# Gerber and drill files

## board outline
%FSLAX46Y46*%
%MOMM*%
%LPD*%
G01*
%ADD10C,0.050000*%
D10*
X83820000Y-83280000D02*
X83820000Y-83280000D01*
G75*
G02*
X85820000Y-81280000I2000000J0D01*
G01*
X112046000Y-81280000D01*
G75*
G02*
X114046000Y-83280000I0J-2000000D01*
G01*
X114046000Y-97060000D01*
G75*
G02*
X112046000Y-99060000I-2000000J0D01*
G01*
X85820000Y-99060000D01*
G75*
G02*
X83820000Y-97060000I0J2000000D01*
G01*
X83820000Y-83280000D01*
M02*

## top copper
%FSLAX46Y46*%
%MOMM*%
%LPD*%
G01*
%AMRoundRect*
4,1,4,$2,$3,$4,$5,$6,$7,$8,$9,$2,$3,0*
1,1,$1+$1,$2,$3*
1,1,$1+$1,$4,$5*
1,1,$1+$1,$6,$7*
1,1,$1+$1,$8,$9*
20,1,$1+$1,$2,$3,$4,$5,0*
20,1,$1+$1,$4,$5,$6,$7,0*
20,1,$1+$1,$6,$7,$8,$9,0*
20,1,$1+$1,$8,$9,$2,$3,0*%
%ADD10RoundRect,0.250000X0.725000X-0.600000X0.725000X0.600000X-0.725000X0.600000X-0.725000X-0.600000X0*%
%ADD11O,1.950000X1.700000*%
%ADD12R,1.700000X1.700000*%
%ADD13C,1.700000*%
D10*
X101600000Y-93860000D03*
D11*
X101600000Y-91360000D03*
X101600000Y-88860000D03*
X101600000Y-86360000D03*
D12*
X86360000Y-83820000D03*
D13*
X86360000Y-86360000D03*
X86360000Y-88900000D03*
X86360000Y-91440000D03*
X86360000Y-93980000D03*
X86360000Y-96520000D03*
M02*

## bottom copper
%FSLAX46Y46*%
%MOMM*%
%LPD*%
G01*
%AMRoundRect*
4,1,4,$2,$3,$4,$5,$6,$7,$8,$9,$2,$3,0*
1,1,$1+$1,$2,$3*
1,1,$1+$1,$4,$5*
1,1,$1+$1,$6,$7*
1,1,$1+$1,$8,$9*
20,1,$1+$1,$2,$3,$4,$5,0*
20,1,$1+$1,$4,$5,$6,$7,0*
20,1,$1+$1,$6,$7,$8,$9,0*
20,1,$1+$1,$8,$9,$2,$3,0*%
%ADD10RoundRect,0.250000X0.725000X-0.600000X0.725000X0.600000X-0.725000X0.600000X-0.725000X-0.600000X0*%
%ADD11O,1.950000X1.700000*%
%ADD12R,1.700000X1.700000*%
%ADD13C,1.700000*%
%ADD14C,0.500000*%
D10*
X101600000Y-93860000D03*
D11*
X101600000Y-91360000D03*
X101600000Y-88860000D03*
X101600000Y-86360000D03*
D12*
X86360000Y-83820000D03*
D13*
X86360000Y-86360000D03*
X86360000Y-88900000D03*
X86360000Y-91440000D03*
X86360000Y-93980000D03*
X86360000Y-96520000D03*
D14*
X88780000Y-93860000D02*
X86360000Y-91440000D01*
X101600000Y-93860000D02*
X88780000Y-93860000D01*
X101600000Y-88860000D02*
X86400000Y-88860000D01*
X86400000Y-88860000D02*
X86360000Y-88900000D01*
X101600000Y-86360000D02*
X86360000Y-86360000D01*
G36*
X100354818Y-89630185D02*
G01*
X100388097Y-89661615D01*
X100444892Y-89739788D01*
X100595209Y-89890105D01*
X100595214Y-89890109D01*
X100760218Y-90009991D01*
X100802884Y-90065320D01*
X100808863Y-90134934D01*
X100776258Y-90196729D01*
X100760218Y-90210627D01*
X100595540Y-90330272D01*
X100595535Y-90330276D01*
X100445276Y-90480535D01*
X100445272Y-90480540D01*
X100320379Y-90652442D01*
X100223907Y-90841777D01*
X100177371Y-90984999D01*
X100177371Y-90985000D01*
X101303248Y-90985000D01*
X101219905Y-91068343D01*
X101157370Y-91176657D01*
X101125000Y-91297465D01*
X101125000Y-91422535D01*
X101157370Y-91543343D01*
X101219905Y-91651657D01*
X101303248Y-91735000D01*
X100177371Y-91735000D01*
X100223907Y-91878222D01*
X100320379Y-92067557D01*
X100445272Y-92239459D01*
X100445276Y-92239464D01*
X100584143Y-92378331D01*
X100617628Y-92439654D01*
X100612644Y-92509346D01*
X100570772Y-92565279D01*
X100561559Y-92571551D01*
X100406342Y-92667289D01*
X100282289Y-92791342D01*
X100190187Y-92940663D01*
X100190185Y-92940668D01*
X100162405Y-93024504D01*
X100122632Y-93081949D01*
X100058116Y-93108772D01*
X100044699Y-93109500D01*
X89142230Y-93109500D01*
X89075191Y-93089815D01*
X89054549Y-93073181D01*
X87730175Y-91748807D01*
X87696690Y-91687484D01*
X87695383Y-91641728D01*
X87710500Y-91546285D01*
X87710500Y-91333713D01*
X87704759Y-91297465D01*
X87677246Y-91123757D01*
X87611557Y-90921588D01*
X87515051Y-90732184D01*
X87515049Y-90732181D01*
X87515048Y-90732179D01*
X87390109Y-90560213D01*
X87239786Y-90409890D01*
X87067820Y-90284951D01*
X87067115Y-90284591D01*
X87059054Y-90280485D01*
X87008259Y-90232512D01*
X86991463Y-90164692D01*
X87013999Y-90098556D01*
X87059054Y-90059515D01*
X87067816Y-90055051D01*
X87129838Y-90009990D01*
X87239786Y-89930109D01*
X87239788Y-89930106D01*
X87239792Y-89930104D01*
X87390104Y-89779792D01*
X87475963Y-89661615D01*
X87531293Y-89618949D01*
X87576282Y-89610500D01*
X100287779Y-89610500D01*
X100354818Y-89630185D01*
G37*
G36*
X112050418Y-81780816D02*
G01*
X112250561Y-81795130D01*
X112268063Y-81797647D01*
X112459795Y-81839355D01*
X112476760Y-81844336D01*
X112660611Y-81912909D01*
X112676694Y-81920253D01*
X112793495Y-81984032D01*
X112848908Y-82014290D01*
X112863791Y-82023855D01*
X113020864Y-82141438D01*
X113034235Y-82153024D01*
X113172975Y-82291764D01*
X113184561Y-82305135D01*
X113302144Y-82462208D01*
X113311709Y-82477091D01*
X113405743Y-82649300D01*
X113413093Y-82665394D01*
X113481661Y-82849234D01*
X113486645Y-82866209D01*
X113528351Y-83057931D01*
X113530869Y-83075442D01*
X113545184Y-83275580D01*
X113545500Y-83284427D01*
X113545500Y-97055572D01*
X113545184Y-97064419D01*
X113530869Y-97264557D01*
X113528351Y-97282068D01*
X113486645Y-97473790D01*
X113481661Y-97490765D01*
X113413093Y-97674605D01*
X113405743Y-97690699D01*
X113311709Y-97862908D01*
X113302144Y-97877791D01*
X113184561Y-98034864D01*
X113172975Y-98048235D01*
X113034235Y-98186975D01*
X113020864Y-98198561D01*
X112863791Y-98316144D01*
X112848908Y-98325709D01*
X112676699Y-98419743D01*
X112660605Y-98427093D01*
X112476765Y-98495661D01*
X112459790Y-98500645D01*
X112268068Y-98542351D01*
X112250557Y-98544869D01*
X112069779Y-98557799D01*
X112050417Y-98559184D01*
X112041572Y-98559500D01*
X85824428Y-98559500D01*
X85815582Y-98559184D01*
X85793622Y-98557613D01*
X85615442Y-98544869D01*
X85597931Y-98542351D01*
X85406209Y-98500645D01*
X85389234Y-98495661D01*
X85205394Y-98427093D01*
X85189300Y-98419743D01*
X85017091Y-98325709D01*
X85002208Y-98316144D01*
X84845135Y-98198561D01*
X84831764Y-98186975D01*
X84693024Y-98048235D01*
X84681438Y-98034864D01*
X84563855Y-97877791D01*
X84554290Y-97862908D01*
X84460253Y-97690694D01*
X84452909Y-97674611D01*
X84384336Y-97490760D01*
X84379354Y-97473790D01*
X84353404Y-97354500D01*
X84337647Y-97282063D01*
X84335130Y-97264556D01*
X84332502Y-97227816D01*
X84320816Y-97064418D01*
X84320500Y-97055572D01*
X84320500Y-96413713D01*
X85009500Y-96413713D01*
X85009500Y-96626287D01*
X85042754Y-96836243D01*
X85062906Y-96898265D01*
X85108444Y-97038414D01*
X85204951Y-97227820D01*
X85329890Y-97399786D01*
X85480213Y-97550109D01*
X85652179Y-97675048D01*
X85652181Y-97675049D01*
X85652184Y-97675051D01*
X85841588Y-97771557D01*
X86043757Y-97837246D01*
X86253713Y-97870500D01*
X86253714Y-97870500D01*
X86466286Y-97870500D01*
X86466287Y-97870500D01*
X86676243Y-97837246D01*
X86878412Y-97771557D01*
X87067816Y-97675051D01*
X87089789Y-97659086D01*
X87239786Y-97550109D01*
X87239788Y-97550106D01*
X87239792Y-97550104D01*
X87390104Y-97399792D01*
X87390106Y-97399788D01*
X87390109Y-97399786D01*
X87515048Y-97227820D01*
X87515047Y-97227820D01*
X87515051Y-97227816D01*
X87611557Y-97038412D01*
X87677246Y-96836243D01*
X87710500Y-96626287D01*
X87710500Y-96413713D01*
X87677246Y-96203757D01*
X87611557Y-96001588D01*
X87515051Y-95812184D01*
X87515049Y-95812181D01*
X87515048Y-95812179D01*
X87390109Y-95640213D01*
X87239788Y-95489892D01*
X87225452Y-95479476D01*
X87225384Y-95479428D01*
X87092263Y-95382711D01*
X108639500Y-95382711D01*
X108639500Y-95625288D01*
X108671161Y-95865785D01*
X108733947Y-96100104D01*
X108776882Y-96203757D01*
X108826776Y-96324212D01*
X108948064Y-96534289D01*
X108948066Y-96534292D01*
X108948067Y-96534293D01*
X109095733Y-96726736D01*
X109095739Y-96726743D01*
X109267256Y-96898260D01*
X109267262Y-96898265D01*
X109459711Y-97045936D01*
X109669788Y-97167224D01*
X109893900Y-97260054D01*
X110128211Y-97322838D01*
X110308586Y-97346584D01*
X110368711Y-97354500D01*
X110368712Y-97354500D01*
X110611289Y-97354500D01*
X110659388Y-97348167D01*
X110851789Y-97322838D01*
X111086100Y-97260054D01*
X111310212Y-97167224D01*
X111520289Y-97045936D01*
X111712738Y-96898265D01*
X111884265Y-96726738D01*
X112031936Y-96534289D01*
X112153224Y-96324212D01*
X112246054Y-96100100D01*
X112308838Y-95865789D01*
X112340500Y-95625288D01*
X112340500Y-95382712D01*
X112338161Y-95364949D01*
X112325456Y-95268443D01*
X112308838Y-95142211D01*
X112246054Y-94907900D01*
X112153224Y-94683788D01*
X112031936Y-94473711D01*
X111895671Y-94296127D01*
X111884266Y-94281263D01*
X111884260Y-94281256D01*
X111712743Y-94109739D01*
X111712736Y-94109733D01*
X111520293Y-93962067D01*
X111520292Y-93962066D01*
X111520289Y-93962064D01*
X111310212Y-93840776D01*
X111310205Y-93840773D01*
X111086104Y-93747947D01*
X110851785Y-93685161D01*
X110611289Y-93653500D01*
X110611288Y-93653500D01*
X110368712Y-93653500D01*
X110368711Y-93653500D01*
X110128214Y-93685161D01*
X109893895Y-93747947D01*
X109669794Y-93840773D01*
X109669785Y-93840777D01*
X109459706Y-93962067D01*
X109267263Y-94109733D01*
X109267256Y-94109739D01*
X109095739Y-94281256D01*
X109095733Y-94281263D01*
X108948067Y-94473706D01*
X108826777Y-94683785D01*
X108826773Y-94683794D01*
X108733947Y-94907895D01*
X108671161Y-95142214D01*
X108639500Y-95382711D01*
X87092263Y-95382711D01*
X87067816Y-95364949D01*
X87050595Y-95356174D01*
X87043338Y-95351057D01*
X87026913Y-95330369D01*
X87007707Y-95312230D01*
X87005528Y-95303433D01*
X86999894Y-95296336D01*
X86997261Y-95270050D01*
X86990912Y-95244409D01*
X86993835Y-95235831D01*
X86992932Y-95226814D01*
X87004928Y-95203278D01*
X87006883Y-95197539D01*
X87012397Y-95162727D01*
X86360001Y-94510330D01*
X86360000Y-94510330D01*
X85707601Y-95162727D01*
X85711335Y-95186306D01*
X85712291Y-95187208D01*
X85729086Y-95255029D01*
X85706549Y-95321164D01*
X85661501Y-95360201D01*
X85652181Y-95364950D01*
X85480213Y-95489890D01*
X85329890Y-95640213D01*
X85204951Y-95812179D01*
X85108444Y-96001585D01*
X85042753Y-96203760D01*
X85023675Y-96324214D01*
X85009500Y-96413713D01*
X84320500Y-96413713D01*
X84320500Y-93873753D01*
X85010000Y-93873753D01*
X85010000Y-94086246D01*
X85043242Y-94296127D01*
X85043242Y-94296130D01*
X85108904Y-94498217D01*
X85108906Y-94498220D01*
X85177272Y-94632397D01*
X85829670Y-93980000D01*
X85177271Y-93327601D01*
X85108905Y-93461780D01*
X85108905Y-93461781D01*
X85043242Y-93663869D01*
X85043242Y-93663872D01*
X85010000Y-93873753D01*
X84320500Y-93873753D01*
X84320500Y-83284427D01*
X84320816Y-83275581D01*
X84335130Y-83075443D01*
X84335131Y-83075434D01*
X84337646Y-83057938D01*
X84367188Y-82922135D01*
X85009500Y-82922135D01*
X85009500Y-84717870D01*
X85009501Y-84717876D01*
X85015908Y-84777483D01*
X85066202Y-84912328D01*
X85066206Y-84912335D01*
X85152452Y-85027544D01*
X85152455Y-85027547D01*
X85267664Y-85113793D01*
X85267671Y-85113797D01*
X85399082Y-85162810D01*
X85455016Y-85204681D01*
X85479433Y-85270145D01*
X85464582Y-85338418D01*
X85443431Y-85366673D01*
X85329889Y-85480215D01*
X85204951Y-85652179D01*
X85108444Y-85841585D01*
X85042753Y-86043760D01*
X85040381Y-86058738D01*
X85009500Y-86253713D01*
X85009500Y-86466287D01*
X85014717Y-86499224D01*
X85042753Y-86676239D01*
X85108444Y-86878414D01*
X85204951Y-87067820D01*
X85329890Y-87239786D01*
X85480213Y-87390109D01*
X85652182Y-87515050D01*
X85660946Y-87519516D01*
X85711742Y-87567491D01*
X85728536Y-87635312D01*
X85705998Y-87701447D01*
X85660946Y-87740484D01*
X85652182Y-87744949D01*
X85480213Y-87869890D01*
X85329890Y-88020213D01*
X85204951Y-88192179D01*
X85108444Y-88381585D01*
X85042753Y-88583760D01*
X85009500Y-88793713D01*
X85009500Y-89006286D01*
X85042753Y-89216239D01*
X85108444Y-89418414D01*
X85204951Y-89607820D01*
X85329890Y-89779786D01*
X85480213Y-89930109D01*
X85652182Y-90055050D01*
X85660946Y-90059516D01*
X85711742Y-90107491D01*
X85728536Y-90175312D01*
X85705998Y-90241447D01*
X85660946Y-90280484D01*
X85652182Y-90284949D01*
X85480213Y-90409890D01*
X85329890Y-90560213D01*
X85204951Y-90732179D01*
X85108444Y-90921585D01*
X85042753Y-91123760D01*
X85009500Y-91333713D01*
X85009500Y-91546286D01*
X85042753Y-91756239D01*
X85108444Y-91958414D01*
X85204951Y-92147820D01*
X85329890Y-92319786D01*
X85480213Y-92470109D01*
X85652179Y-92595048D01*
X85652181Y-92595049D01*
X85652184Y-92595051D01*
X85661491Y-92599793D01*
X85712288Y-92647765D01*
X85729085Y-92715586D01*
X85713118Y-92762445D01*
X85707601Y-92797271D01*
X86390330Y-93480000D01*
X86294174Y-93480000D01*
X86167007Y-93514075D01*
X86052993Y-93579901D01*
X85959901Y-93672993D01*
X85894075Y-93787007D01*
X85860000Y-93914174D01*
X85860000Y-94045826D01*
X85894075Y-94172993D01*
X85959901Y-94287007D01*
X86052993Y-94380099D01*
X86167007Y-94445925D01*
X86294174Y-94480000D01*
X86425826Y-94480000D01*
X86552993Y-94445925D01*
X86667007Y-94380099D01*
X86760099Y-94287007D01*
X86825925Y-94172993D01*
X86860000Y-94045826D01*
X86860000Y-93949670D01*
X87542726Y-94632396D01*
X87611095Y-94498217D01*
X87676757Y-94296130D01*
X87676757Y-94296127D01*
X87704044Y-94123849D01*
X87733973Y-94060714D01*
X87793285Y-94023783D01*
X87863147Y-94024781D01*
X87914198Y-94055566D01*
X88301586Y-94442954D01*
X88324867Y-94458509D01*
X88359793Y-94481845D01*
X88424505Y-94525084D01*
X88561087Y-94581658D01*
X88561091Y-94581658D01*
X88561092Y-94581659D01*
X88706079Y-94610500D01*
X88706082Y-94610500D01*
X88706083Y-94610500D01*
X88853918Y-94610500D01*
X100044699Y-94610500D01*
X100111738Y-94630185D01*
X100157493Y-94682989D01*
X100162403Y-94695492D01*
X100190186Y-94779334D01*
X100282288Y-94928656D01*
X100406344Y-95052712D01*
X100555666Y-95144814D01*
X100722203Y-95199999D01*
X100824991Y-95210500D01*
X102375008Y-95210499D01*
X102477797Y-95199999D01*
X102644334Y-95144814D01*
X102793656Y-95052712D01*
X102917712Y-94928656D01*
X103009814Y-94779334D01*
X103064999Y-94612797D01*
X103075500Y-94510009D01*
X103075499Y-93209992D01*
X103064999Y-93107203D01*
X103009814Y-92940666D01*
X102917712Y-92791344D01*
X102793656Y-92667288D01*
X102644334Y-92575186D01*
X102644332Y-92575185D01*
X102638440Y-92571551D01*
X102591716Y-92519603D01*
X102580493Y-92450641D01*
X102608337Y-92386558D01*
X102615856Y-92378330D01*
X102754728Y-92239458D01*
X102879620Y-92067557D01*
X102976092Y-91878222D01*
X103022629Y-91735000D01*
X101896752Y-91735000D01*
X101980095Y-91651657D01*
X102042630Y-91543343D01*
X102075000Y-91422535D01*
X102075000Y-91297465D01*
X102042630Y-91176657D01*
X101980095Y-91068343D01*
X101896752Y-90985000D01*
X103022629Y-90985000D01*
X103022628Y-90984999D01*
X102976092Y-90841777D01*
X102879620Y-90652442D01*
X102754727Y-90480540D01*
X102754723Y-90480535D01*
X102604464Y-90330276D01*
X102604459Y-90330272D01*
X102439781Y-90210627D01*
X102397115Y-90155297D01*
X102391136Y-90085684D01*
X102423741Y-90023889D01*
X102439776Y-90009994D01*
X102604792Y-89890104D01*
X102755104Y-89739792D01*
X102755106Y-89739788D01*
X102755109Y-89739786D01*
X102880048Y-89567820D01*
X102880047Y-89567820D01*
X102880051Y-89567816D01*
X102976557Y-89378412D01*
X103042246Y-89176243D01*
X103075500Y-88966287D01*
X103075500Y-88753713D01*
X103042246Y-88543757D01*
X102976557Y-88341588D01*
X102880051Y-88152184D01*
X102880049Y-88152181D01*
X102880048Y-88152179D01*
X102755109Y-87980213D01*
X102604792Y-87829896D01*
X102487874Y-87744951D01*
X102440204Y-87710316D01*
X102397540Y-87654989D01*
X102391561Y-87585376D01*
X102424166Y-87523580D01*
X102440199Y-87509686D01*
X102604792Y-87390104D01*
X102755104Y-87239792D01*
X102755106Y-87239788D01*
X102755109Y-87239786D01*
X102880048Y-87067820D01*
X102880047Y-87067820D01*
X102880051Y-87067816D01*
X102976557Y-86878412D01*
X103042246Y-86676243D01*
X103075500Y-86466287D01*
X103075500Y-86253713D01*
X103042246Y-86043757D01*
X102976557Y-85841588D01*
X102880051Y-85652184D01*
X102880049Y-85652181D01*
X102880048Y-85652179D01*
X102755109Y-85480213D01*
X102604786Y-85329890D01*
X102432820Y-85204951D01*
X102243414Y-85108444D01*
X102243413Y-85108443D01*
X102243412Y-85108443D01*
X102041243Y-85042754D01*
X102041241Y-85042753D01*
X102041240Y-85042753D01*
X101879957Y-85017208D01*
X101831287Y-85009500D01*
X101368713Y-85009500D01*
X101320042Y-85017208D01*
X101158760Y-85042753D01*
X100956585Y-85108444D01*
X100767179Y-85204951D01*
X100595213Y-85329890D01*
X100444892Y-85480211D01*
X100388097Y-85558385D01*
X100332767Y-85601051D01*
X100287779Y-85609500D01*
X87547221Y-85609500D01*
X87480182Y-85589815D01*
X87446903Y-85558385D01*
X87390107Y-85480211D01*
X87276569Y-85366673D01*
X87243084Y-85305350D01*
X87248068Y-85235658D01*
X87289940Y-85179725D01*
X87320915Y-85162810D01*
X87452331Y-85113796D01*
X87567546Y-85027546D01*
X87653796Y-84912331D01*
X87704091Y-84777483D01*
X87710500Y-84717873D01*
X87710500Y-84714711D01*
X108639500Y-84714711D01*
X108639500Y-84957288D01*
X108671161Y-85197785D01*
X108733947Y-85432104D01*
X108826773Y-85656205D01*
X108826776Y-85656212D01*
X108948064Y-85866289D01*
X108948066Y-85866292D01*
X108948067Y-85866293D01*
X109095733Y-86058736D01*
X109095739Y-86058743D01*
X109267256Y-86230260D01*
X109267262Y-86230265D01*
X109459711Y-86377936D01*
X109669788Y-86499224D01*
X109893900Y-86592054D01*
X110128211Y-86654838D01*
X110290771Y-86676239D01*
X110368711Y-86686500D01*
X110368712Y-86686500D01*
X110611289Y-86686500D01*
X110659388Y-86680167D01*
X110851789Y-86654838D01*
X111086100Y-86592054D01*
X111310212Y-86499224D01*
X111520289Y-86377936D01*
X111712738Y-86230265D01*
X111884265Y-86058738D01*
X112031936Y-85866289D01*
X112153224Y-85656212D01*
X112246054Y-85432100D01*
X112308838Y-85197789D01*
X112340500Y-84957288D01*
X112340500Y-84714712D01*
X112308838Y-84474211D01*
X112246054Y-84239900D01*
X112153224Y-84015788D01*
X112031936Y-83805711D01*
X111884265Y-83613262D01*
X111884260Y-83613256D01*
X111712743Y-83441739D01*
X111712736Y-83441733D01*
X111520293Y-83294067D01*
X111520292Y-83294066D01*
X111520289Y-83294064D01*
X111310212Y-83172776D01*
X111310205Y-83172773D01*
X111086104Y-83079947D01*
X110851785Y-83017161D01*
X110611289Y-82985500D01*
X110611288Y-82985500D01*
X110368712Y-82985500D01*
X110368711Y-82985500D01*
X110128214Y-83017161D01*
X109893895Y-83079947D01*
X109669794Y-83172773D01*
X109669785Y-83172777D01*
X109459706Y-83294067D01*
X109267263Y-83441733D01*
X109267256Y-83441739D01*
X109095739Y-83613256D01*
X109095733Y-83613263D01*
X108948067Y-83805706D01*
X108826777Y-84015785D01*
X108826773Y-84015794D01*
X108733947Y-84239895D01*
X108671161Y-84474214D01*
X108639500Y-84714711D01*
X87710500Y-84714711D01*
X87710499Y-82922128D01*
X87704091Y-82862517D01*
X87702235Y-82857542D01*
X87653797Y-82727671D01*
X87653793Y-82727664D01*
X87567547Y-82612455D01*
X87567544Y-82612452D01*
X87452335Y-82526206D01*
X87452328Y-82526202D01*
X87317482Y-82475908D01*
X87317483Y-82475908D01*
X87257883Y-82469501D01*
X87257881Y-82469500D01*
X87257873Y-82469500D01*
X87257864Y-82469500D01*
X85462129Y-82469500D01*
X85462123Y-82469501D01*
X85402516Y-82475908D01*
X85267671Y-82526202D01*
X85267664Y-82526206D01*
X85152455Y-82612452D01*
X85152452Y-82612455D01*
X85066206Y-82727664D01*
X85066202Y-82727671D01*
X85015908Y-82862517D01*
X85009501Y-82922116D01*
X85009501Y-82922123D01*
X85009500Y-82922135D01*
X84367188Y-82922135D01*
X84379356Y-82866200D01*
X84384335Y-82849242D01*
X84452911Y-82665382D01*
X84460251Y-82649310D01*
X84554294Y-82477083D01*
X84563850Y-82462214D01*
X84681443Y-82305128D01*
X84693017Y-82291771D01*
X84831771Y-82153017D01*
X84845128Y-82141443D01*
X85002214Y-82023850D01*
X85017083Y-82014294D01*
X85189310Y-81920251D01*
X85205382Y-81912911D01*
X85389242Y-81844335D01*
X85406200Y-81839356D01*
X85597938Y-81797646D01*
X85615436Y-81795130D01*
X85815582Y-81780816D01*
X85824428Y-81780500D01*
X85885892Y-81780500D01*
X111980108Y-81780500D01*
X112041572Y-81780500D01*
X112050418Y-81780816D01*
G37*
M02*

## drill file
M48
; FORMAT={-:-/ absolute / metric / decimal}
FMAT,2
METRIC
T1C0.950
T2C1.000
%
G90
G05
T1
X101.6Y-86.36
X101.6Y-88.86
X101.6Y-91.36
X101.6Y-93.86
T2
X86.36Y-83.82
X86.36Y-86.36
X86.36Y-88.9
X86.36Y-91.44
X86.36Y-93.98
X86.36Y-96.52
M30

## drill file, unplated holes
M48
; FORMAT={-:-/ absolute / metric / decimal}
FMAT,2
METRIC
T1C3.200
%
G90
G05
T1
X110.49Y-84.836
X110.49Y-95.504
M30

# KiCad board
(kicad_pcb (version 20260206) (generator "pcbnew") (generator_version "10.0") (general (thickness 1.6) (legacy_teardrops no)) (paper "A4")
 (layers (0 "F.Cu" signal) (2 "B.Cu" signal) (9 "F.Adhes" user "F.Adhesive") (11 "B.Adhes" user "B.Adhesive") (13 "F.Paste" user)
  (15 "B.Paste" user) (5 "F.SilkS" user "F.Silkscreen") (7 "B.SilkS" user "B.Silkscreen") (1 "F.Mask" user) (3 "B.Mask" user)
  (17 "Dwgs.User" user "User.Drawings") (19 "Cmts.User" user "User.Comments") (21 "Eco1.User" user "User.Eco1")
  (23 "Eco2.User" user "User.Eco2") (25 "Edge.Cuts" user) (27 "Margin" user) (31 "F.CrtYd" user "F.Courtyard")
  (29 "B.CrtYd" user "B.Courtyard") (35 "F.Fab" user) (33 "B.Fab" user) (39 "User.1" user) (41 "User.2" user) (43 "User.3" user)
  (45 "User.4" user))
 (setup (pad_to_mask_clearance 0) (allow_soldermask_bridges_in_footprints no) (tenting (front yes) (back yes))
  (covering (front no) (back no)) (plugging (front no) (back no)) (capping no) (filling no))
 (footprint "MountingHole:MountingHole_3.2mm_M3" (layer "F.Cu") (at 110.49 95.504)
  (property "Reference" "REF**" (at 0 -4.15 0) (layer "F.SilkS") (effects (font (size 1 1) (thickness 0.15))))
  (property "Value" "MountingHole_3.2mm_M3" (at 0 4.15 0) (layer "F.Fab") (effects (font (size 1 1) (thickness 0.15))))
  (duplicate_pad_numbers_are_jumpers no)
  (pad "" np_thru_hole circle (at 0 0) (size 3.2 3.2) (drill 3.2) (layers "*.Cu" "*.Mask")))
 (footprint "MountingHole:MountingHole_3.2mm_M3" (layer "F.Cu") (at 110.49 84.836)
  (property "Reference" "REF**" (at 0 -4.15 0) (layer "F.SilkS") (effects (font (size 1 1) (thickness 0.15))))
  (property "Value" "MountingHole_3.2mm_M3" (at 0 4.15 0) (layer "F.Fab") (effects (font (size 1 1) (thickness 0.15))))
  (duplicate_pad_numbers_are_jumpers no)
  (pad "" np_thru_hole circle (at 0 0) (size 3.2 3.2) (drill 3.2) (layers "*.Cu" "*.Mask")))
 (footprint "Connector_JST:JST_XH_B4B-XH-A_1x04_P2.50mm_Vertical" (layer "F.Cu") (at 101.6 93.86 90)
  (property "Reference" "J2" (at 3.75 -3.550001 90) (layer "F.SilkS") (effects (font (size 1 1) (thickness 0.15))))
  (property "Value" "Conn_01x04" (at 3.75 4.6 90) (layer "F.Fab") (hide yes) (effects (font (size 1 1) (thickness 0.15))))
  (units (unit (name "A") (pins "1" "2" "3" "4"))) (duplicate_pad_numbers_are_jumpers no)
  (pad "1" thru_hole roundrect (at 0 0 90) (size 1.7 1.95) (drill 0.95) (layers "*.Cu" "*.Mask") (remove_unused_layers no)
   (roundrect_rratio 0.147059) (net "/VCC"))
  (pad "2" thru_hole oval (at 2.5 0 90) (size 1.7 1.95) (drill 0.95) (layers "*.Cu" "*.Mask") (remove_unused_layers no) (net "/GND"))
  (pad "3" thru_hole oval (at 5 0 90) (size 1.7 1.95) (drill 0.95) (layers "*.Cu" "*.Mask") (remove_unused_layers no) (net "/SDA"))
  (pad "4" thru_hole oval (at 7.5 0 90) (size 1.7 1.95) (drill 0.95) (layers "*.Cu" "*.Mask") (remove_unused_layers no) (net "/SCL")))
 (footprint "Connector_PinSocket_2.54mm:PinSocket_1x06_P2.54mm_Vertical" (layer "F.Cu") (at 86.36 83.82)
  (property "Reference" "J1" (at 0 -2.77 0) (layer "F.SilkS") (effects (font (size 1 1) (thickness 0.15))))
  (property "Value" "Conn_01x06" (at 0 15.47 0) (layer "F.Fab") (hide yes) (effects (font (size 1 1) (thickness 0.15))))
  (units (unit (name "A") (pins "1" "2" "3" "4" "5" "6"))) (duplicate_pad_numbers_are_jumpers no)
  (pad "1" thru_hole rect (at 0 0) (size 1.7 1.7) (drill 1) (layers "*.Cu" "*.Mask") (remove_unused_layers no) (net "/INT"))
  (pad "2" thru_hole circle (at 0 2.54) (size 1.7 1.7) (drill 1) (layers "*.Cu" "*.Mask") (remove_unused_layers no) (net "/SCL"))
  (pad "3" thru_hole circle (at 0 5.08) (size 1.7 1.7) (drill 1) (layers "*.Cu" "*.Mask") (remove_unused_layers no) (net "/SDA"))
  (pad "4" thru_hole circle (at 0 7.62) (size 1.7 1.7) (drill 1) (layers "*.Cu" "*.Mask") (remove_unused_layers no) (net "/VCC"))
  (pad "5" thru_hole circle (at 0 10.16) (size 1.7 1.7) (drill 1) (layers "*.Cu" "*.Mask") (remove_unused_layers no) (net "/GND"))
  (pad "6" thru_hole circle (at 0 12.7) (size 1.7 1.7) (drill 1) (layers "*.Cu" "*.Mask") (remove_unused_layers no) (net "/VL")))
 (gr_rect (start 83.82 81.28) (end 114.046 99.06) (radius 2) (stroke (width 0.05) (type solid)) (fill no) (layer "Edge.Cuts"))
 (segment (start 88.78 93.86) (end 86.36 91.44) (width 0.5) (layer "B.Cu") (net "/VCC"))
 (segment (start 101.6 93.86) (end 88.78 93.86) (width 0.5) (layer "B.Cu") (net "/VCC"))
 (segment (start 101.6 88.86) (end 86.4 88.86) (width 0.5) (layer "B.Cu") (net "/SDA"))
 (segment (start 86.4 88.86) (end 86.36 88.9) (width 0.5) (layer "B.Cu") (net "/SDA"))
 (segment (start 101.6 86.36) (end 86.36 86.36) (width 0.5) (layer "B.Cu") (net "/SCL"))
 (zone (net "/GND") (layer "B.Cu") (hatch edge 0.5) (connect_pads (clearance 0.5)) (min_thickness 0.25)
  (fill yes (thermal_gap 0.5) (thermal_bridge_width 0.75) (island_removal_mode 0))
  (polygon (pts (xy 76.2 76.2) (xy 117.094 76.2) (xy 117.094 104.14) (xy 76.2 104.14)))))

